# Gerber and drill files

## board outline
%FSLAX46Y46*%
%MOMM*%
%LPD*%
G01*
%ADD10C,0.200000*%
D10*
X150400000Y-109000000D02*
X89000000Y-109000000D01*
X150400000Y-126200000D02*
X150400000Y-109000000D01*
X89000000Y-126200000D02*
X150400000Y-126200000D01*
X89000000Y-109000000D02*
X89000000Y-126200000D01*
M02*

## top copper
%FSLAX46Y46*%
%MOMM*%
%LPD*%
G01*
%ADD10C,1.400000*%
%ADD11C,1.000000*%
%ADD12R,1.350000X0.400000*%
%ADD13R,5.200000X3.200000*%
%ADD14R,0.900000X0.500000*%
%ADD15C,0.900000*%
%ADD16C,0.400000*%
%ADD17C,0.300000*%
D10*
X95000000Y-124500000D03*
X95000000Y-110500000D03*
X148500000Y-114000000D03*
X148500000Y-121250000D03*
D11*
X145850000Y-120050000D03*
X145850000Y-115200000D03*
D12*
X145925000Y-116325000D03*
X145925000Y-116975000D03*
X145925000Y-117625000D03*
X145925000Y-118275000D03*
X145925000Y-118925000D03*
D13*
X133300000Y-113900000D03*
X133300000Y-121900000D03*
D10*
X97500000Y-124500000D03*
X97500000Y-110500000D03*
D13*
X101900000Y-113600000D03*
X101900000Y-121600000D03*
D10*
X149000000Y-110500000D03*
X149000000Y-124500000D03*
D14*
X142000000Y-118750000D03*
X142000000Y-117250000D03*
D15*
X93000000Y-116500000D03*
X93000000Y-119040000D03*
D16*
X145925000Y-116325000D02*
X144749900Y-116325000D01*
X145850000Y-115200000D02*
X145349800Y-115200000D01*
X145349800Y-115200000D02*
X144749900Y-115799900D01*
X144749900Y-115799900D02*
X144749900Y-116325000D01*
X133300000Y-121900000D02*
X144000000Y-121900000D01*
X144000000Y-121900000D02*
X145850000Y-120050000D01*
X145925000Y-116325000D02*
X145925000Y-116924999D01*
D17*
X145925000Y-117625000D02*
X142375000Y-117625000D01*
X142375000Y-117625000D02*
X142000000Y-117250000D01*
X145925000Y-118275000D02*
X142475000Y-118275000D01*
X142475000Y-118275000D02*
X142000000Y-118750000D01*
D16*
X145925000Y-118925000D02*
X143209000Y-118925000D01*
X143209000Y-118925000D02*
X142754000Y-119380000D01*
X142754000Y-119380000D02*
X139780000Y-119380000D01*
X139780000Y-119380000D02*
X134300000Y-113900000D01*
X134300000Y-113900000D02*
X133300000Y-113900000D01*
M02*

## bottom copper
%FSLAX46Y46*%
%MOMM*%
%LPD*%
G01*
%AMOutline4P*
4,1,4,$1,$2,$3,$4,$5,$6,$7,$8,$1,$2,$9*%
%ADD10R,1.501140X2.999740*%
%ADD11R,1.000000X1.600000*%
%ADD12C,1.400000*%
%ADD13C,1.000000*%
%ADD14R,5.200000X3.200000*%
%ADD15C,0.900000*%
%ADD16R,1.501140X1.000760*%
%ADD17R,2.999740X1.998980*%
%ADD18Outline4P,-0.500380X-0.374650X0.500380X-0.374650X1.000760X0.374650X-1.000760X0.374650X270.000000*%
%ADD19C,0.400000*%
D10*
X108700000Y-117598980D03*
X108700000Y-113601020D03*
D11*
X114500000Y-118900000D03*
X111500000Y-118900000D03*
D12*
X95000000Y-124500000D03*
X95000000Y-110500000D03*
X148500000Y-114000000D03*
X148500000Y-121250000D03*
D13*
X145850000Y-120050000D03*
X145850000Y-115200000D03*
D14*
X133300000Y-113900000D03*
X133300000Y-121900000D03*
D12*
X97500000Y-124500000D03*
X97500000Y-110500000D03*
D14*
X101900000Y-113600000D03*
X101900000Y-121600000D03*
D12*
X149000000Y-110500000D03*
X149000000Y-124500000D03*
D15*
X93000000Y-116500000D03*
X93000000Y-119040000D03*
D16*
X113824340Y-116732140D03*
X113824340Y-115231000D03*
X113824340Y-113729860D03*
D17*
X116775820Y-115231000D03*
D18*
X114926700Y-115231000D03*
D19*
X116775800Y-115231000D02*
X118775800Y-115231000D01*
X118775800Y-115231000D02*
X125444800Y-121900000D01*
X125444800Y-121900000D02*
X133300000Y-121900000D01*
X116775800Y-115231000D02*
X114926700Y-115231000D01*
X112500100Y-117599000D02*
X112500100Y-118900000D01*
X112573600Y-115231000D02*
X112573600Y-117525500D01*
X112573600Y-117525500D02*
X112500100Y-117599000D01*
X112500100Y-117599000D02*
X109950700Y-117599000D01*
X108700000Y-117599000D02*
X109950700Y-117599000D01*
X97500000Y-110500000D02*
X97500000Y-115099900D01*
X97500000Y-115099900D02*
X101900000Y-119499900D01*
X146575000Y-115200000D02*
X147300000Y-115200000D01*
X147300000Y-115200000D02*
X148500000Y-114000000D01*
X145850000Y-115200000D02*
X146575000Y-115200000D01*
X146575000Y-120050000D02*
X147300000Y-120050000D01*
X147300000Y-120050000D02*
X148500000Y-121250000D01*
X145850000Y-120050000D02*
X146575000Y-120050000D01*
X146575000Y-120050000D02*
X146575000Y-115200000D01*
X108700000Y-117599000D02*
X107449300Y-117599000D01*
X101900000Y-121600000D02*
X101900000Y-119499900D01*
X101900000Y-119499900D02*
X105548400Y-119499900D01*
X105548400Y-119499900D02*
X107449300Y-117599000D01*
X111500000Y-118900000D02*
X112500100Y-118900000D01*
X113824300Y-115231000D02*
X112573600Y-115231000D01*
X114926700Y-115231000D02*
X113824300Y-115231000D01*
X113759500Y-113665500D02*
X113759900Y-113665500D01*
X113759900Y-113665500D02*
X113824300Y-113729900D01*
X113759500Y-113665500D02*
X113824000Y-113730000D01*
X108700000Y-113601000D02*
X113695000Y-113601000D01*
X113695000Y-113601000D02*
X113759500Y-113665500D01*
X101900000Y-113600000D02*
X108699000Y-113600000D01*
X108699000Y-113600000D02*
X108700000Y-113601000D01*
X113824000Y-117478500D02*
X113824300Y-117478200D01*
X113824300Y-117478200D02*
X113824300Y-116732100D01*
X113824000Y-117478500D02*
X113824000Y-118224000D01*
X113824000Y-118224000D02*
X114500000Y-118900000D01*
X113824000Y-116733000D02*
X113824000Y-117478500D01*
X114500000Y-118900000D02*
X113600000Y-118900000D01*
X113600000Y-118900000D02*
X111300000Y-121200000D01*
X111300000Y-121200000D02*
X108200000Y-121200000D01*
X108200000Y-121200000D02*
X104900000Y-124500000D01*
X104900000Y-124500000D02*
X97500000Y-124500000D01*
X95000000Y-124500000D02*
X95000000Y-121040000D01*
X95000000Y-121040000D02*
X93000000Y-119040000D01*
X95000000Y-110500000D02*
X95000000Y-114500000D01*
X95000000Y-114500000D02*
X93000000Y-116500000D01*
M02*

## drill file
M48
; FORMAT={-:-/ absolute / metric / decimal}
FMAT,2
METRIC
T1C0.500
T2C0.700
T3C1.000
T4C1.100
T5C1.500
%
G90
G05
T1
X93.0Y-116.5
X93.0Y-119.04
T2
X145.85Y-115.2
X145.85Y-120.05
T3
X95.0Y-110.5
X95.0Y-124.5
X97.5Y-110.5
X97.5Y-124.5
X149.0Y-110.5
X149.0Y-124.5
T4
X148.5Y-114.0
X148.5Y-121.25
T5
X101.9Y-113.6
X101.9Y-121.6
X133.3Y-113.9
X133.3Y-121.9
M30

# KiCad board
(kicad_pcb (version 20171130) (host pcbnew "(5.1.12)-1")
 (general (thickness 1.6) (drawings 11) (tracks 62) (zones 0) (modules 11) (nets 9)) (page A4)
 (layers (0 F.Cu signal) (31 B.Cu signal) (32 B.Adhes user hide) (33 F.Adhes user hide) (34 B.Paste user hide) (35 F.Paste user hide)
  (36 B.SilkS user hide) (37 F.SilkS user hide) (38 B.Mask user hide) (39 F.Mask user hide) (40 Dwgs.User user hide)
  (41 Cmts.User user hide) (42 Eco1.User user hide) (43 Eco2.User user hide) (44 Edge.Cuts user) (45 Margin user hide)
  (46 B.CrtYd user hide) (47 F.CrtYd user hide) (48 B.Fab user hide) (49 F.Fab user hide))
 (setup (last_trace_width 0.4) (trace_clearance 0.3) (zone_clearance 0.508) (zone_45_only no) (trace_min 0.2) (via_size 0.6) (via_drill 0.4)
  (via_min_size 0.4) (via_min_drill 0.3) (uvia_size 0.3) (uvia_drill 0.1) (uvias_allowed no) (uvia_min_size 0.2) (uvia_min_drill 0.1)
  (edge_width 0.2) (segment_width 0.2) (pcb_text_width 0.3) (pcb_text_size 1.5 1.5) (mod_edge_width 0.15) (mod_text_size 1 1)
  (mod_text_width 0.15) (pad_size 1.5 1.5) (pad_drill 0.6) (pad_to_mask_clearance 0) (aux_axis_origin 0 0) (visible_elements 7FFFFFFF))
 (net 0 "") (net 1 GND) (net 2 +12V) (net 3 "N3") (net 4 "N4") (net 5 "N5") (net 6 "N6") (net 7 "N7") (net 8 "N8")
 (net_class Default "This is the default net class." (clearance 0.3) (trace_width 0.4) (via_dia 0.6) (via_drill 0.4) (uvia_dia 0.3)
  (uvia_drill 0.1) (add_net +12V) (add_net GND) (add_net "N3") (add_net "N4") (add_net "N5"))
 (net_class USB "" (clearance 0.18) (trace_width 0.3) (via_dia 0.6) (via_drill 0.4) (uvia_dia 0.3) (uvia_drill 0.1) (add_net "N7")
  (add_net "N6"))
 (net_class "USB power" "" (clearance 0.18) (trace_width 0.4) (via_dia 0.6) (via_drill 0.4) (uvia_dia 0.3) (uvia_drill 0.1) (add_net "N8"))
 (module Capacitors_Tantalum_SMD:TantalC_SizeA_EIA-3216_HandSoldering (layer B.Cu) (at 108.7 115.6 270)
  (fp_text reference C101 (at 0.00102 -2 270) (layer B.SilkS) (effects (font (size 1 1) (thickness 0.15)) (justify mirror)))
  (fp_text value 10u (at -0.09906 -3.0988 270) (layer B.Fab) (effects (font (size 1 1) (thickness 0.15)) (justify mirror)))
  (pad 2 smd rect (at 1.99898 0 270) (size 2.99974 1.50114) (layers B.Cu B.Paste B.Mask) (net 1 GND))
  (pad 1 smd rect (at -1.99898 0 270) (size 2.99974 1.50114) (layers B.Cu B.Paste B.Mask) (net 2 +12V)))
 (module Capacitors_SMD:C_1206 (layer B.Cu) (at 113 118.9 180)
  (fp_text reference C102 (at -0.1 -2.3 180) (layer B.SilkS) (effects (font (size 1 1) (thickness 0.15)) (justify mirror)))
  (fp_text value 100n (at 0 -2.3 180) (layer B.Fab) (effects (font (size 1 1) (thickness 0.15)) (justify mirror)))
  (pad 1 smd rect (at -1.5 0 180) (size 1 1.6) (layers B.Cu B.Paste B.Mask) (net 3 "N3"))
  (pad 2 smd rect (at 1.5 0 180) (size 1 1.6) (layers B.Cu B.Paste B.Mask) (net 1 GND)))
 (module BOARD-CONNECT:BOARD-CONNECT (layer F.Cu) (at 95 125 180)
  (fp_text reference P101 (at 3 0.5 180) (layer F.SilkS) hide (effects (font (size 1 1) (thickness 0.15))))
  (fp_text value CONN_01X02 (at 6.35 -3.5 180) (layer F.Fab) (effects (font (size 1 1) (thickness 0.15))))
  (pad 1 thru_hole circle (at 0 0.5 180) (size 1.4 1.4) (drill 1) (layers *.Cu *.Mask) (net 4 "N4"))
  (pad 2 thru_hole circle (at 0 14.5 180) (size 1.4 1.4) (drill 1) (layers *.Cu *.Mask) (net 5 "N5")))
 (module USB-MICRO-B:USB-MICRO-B (layer F.Cu) (at 148.5 114 270)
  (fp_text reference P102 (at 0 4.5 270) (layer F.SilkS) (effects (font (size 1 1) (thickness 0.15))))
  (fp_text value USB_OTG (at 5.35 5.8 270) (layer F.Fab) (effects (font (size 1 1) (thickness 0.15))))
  (pad 6 thru_hole circle (at 0 0 270) (size 1.4 1.4) (drill 1.1) (layers *.Cu *.Mask) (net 1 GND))
  (pad 6 thru_hole circle (at 7.25 0 270) (size 1.4 1.4) (drill 1.1) (layers *.Cu *.Mask) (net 1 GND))
  (pad 6 thru_hole circle (at 6.05 2.65 270) (size 1 1) (drill 0.7) (layers *.Cu *.Mask) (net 1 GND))
  (pad 6 thru_hole circle (at 1.2 2.65 270) (size 1 1) (drill 0.7) (layers *.Cu *.Mask) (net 1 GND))
  (pad 5 smd rect (at 2.325 2.575 270) (size 0.4 1.35) (layers F.Cu F.Paste F.Mask) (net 1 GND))
  (pad 4 smd rect (at 2.975 2.575 270) (size 0.4 1.35) (layers F.Cu F.Paste F.Mask) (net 1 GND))
  (pad 3 smd rect (at 3.625 2.575 270) (size 0.4 1.35) (layers F.Cu F.Paste F.Mask) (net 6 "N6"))
  (pad 2 smd rect (at 4.275 2.575 270) (size 0.4 1.35) (layers F.Cu F.Paste F.Mask) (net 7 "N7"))
  (pad 1 smd rect (at 4.925 2.575 270) (size 0.4 1.35) (layers F.Cu F.Paste F.Mask) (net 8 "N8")))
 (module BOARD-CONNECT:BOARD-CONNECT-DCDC (layer F.Cu) (at 133.3 113.9)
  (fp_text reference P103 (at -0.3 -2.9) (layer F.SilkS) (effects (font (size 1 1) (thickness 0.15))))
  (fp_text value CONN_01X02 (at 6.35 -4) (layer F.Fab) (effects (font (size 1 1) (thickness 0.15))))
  (pad 1 thru_hole rect (at 0 0) (size 5.2 3.2) (drill 1.5) (layers *.Cu *.Mask) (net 8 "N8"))
  (pad 2 thru_hole rect (at 0 8) (size 5.2 3.2) (drill 1.5) (layers *.Cu *.Mask) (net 1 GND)))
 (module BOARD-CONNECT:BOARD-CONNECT (layer F.Cu) (at 97.5 125 180)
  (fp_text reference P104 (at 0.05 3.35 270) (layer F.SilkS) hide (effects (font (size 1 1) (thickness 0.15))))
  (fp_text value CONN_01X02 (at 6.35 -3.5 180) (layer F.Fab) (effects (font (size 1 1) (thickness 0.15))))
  (pad 1 thru_hole circle (at 0 0.5 180) (size 1.4 1.4) (drill 1) (layers *.Cu *.Mask) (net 3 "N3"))
  (pad 2 thru_hole circle (at 0 14.5 180) (size 1.4 1.4) (drill 1) (layers *.Cu *.Mask) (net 1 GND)))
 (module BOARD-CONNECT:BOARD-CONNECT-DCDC (layer F.Cu) (at 101.9 113.6)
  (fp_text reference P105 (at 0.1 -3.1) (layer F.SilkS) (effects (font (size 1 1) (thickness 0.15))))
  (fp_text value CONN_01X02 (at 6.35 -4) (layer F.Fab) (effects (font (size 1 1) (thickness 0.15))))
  (pad 1 thru_hole rect (at 0 0) (size 5.2 3.2) (drill 1.5) (layers *.Cu *.Mask) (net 2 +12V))
  (pad 2 thru_hole rect (at 0 8) (size 5.2 3.2) (drill 1.5) (layers *.Cu *.Mask) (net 1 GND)))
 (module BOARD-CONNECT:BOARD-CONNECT (layer F.Cu) (at 149 110)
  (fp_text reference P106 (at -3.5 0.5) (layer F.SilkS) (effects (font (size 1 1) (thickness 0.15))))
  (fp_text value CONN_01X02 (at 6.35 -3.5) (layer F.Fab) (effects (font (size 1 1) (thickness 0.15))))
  (pad 1 thru_hole circle (at 0 0.5) (size 1.4 1.4) (drill 1) (layers *.Cu *.Mask))
  (pad 2 thru_hole circle (at 0 14.5) (size 1.4 1.4) (drill 1) (layers *.Cu *.Mask)))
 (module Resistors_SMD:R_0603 (layer F.Cu) (at 142 118 90)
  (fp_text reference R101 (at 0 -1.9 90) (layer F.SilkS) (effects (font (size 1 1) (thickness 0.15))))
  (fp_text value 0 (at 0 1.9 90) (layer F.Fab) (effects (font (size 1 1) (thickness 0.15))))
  (pad 1 smd rect (at -0.75 0 90) (size 0.5 0.9) (layers F.Cu F.Paste F.Mask) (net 7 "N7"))
  (pad 2 smd rect (at 0.75 0 90) (size 0.5 0.9) (layers F.Cu F.Paste F.Mask) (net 6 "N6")))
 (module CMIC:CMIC (layer F.Cu) (at 93 122.52 90)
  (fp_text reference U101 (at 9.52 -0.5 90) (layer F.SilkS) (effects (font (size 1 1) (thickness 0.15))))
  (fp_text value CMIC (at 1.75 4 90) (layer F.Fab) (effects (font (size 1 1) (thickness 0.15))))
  (pad 2 thru_hole circle (at 6.02 0 90) (size 0.9 0.9) (drill 0.5) (layers *.Cu *.Mask) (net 5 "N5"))
  (pad 1 thru_hole circle (at 3.48 0 90) (size 0.9 0.9) (drill 0.5) (layers *.Cu *.Mask) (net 4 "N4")))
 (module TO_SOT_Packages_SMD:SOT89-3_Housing (layer B.Cu) (at 115.676 115.231 90)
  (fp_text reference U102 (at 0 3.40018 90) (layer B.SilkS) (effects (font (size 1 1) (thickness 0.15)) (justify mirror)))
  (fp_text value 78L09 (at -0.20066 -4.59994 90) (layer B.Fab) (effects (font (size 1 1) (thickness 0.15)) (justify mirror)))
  (pad 1 smd rect (at -1.50114 -1.85166 90) (size 1.00076 1.50114) (layers B.Cu B.Paste B.Mask) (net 3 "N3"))
  (pad 2 smd rect (at 0 -1.85166 90) (size 1.00076 1.50114) (layers B.Cu B.Paste B.Mask) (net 1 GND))
  (pad 3 smd rect (at 1.50114 -1.85166 90) (size 1.00076 1.50114) (layers B.Cu B.Paste B.Mask) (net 2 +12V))
  (pad 2 smd rect (at 0 1.09982 90) (size 1.99898 2.99974) (layers B.Cu B.Paste B.Mask) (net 1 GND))
  (pad 2 smd trapezoid (at 0 -0.7493 270) (size 1.50114 0.7493) (rect_delta 0 -0.50038) (layers B.Cu B.Paste B.Mask) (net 1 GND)))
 (gr_line (start 150.4 109) (end 89 109) (layer Edge.Cuts) (width 0.2))
 (gr_line (start 150.4 126.2) (end 150.4 109) (layer Edge.Cuts) (width 0.2))
 (gr_line (start 89 126.2) (end 150.4 126.2) (layer Edge.Cuts) (width 0.2))
 (gr_line (start 89 109) (end 89 126.2) (layer Edge.Cuts) (width 0.2))
 (segment (start 145.925 116.325) (end 144.7499 116.325) (width 0.4) (layer F.Cu) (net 1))
 (segment (start 116.7758 115.231) (end 118.7758 115.231) (width 0.4) (layer B.Cu) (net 1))
 (segment (start 118.7758 115.231) (end 125.4448 121.9) (width 0.4) (layer B.Cu) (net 1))
 (segment (start 125.4448 121.9) (end 133.3 121.9) (width 0.4) (layer B.Cu) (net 1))
 (segment (start 116.7758 115.231) (end 114.9267 115.231) (width 0.4) (layer B.Cu) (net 1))
 (segment (start 112.5001 117.599) (end 112.5001 118.9) (width 0.4) (layer B.Cu) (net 1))
 (segment (start 112.5736 115.231) (end 112.5736 117.5255) (width 0.4) (layer B.Cu) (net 1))
 (segment (start 112.5736 117.5255) (end 112.5001 117.599) (width 0.4) (layer B.Cu) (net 1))
 (segment (start 112.5001 117.599) (end 109.9507 117.599) (width 0.4) (layer B.Cu) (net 1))
 (segment (start 108.7 117.599) (end 109.9507 117.599) (width 0.4) (layer B.Cu) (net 1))
 (segment (start 97.5 110.5) (end 97.5 115.0999) (width 0.4) (layer B.Cu) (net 1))
 (segment (start 97.5 115.0999) (end 101.9 119.4999) (width 0.4) (layer B.Cu) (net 1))
 (segment (start 145.85 115.2) (end 145.3498 115.2) (width 0.4) (layer F.Cu) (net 1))
 (segment (start 145.3498 115.2) (end 144.7499 115.7999) (width 0.4) (layer F.Cu) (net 1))
 (segment (start 144.7499 115.7999) (end 144.7499 116.325) (width 0.4) (layer F.Cu) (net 1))
 (segment (start 146.575 115.2) (end 147.3 115.2) (width 0.4) (layer B.Cu) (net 1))
 (segment (start 147.3 115.2) (end 148.5 114) (width 0.4) (layer B.Cu) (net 1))
 (segment (start 145.85 115.2) (end 146.575 115.2) (width 0.4) (layer B.Cu) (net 1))
 (segment (start 146.575 120.05) (end 147.3 120.05) (width 0.4) (layer B.Cu) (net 1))
 (segment (start 147.3 120.05) (end 148.5 121.25) (width 0.4) (layer B.Cu) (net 1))
 (segment (start 145.85 120.05) (end 146.575 120.05) (width 0.4) (layer B.Cu) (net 1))
 (segment (start 146.575 120.05) (end 146.575 115.2) (width 0.4) (layer B.Cu) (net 1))
 (segment (start 133.3 121.9) (end 144 121.9) (width 0.4) (layer F.Cu) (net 1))
 (segment (start 144 121.9) (end 145.85 120.05) (width 0.4) (layer F.Cu) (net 1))
 (segment (start 108.7 117.599) (end 107.4493 117.599) (width 0.4) (layer B.Cu) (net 1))
 (segment (start 101.9 121.6) (end 101.9 119.4999) (width 0.4) (layer B.Cu) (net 1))
 (segment (start 101.9 119.4999) (end 105.5484 119.4999) (width 0.4) (layer B.Cu) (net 1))
 (segment (start 105.5484 119.4999) (end 107.4493 117.599) (width 0.4) (layer B.Cu) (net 1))
 (segment (start 111.5 118.9) (end 112.5001 118.9) (width 0.4) (layer B.Cu) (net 1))
 (segment (start 113.8243 115.231) (end 112.5736 115.231) (width 0.4) (layer B.Cu) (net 1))
 (segment (start 114.9267 115.231) (end 113.8243 115.231) (width 0.4) (layer B.Cu) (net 1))
 (segment (start 145.925 116.325) (end 145.925 116.924999) (width 0.4) (layer F.Cu) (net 1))
 (segment (start 113.7595 113.6655) (end 113.7599 113.6655) (width 0.4) (layer B.Cu) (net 2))
 (segment (start 113.7599 113.6655) (end 113.8243 113.7299) (width 0.4) (layer B.Cu) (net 2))
 (segment (start 113.7595 113.6655) (end 113.824 113.73) (width 0.4) (layer B.Cu) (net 2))
 (segment (start 108.7 113.601) (end 113.695 113.601) (width 0.4) (layer B.Cu) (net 2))
 (segment (start 113.695 113.601) (end 113.7595 113.6655) (width 0.4) (layer B.Cu) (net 2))
 (segment (start 101.9 113.6) (end 108.699 113.6) (width 0.4) (layer B.Cu) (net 2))
 (segment (start 108.699 113.6) (end 108.7 113.601) (width 0.4) (layer B.Cu) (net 2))
 (segment (start 113.824 117.4785) (end 113.8243 117.4782) (width 0.4) (layer B.Cu) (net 3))
 (segment (start 113.8243 117.4782) (end 113.8243 116.7321) (width 0.4) (layer B.Cu) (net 3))
 (segment (start 113.824 117.4785) (end 113.824 118.224) (width 0.4) (layer B.Cu) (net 3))
 (segment (start 113.824 118.224) (end 114.5 118.9) (width 0.4) (layer B.Cu) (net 3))
 (segment (start 113.824 116.733) (end 113.824 117.4785) (width 0.4) (layer B.Cu) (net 3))
 (segment (start 114.5 118.9) (end 113.6 118.9) (width 0.4) (layer B.Cu) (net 3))
 (segment (start 113.6 118.9) (end 111.3 121.2) (width 0.4) (layer B.Cu) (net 3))
 (segment (start 111.3 121.2) (end 108.2 121.2) (width 0.4) (layer B.Cu) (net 3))
 (segment (start 108.2 121.2) (end 104.9 124.5) (width 0.4) (layer B.Cu) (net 3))
 (segment (start 104.9 124.5) (end 97.5 124.5) (width 0.4) (layer B.Cu) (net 3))
 (segment (start 95 124.5) (end 95 121.04) (width 0.4) (layer B.Cu) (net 4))
 (segment (start 95 121.04) (end 93 119.04) (width 0.4) (layer B.Cu) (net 4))
 (segment (start 95 110.5) (end 95 114.5) (width 0.4) (layer B.Cu) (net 5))
 (segment (start 95 114.5) (end 93 116.5) (width 0.4) (layer B.Cu) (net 5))
 (segment (start 145.925 117.625) (end 142.375 117.625) (width 0.3) (layer F.Cu) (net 6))
 (segment (start 142.375 117.625) (end 142 117.25) (width 0.3) (layer F.Cu) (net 6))
 (segment (start 145.925 118.275) (end 142.475 118.275) (width 0.3) (layer F.Cu) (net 7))
 (segment (start 142.475 118.275) (end 142 118.75) (width 0.3) (layer F.Cu) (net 7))
 (segment (start 145.925 118.925) (end 143.209 118.925) (width 0.4) (layer F.Cu) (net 8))
 (segment (start 143.209 118.925) (end 142.754 119.38) (width 0.4) (layer F.Cu) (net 8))
 (segment (start 142.754 119.38) (end 139.78 119.38) (width 0.4) (layer F.Cu) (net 8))
 (segment (start 139.78 119.38) (end 134.3 113.9) (width 0.4) (layer F.Cu) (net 8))
 (segment (start 134.3 113.9) (end 133.3 113.9) (width 0.4) (layer F.Cu) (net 8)))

